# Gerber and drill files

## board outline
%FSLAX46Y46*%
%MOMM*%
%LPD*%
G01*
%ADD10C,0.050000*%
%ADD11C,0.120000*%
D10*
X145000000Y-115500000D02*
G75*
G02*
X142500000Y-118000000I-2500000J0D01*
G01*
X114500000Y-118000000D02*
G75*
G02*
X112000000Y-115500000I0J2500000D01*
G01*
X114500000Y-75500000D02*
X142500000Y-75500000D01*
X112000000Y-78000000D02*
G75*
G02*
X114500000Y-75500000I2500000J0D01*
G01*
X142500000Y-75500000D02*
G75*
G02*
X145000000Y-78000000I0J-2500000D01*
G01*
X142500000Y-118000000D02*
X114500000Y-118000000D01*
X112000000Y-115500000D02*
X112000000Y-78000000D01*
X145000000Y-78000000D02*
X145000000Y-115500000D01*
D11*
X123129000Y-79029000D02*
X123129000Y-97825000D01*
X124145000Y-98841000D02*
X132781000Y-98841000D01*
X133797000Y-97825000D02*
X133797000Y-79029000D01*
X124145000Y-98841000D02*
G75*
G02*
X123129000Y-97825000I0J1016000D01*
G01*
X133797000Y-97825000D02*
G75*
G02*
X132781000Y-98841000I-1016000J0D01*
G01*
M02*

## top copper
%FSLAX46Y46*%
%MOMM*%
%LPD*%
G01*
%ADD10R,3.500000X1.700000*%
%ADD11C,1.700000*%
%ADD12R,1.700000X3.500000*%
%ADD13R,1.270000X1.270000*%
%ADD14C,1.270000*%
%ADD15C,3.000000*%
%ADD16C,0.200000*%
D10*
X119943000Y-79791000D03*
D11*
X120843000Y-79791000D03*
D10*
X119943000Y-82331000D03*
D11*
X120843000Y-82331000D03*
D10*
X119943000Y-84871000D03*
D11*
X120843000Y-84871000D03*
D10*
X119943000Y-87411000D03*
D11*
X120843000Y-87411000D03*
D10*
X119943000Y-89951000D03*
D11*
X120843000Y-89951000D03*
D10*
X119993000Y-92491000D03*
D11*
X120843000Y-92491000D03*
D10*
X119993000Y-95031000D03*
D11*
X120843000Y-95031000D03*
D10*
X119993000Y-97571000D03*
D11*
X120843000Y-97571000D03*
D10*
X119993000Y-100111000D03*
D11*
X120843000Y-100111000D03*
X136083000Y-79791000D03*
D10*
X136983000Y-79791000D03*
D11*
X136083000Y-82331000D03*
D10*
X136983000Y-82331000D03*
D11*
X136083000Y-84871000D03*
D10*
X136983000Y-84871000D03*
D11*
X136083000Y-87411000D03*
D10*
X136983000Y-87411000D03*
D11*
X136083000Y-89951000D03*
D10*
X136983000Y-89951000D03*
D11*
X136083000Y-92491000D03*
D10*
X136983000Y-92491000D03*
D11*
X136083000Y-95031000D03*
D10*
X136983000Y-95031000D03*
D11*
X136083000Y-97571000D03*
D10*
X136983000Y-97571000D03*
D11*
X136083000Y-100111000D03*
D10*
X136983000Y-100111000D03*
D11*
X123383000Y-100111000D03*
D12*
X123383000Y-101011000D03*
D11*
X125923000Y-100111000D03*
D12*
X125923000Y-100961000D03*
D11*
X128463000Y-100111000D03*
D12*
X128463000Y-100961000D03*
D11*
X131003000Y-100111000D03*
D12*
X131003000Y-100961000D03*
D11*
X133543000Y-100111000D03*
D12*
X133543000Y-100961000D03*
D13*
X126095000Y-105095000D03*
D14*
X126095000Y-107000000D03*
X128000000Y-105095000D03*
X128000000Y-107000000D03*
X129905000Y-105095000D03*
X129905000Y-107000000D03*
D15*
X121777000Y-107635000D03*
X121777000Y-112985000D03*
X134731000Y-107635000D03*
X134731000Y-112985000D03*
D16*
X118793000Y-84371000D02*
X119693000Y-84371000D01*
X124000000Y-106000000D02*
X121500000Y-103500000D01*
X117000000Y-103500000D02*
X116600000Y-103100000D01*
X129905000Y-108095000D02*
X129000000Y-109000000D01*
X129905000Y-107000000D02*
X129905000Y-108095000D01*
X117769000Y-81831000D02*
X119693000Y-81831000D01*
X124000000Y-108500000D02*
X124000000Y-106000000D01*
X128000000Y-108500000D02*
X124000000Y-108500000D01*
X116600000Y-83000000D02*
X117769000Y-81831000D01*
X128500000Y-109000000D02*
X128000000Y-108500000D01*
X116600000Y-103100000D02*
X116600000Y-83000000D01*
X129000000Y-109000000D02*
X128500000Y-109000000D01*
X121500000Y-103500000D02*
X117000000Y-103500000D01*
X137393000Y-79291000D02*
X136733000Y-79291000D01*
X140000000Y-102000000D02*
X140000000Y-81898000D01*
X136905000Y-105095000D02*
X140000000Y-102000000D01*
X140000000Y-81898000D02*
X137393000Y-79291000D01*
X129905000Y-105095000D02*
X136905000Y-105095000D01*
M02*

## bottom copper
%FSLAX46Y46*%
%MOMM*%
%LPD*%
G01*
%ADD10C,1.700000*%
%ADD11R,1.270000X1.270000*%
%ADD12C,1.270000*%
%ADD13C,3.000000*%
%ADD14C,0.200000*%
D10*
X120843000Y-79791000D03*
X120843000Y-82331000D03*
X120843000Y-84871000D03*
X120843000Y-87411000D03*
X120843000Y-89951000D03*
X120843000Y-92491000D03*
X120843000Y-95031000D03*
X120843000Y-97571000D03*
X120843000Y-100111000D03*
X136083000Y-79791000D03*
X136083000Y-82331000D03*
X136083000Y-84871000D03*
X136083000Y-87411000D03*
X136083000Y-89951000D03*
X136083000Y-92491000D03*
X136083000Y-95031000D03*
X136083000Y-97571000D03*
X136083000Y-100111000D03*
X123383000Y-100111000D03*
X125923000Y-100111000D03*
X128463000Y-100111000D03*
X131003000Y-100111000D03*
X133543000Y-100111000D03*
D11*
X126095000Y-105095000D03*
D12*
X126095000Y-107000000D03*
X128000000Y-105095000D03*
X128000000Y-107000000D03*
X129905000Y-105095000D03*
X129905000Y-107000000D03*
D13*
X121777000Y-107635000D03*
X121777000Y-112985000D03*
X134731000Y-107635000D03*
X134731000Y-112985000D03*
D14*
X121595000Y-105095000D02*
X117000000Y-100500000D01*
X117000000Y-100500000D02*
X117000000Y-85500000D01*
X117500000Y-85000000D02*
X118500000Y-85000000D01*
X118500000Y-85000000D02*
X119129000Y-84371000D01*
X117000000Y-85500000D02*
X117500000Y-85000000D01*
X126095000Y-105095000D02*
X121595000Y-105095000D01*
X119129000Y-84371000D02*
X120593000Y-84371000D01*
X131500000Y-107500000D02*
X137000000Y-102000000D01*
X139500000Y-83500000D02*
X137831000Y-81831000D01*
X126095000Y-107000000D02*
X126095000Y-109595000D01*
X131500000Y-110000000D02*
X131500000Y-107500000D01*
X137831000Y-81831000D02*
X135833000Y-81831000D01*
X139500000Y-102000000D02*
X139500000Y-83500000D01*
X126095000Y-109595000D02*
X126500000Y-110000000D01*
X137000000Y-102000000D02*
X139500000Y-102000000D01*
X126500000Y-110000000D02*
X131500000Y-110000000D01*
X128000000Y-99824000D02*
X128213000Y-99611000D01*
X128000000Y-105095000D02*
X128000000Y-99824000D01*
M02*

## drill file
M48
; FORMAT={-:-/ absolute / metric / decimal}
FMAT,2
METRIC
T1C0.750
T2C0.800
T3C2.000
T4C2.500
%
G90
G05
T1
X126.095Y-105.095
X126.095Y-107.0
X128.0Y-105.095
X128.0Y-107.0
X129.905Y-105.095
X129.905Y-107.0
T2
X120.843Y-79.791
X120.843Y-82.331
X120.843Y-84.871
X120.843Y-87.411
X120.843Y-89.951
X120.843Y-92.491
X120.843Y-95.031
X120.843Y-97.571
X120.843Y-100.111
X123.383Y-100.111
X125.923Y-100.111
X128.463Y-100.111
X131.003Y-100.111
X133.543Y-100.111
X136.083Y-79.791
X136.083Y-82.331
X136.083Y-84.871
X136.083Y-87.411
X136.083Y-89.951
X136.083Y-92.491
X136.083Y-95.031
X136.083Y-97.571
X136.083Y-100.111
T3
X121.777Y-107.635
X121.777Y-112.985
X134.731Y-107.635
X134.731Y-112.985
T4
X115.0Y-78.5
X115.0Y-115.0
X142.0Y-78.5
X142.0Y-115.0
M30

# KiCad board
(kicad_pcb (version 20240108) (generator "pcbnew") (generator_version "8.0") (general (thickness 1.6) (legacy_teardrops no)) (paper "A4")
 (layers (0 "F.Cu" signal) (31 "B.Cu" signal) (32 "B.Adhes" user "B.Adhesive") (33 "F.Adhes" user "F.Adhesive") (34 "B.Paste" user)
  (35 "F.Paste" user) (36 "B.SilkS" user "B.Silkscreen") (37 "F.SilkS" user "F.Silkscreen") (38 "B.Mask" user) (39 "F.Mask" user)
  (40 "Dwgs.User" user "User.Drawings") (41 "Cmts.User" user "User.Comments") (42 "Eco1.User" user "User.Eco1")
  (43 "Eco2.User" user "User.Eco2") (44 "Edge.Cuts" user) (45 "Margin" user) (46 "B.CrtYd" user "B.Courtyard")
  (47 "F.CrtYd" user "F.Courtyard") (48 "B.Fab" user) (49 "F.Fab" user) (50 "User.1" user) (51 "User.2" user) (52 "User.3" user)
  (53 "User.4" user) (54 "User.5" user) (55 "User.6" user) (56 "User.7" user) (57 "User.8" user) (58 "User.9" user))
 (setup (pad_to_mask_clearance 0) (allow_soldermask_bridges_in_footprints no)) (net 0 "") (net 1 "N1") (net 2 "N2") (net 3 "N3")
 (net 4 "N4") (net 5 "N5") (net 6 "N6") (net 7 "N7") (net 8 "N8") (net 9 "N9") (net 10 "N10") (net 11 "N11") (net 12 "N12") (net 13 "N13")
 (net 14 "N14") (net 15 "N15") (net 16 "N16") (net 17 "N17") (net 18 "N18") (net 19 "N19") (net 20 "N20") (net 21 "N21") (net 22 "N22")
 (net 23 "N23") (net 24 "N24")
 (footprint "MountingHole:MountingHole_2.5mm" (layer "F.Cu") (at 142 115)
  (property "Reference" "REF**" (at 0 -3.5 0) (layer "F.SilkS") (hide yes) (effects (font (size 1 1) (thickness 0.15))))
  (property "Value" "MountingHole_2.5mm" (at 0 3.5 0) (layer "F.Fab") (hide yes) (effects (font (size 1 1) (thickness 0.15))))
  (pad "" np_thru_hole circle (at 0 0) (size 2.5 2.5) (drill 2.5) (layers "*.Cu" "*.Mask")))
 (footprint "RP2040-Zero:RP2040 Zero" (layer "F.Cu") (at 118.303 102.778)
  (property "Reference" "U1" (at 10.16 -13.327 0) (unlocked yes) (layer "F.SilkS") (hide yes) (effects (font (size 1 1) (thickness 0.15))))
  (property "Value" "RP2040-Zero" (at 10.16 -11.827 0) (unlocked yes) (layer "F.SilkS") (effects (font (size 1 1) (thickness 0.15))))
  (fp_line (start 4.826 -23.749) (end 4.826 -4.953) (stroke (width 0.12) (type default)) (layer "Edge.Cuts"))
  (fp_line (start 5.842 -3.937) (end 14.478 -3.937) (stroke (width 0.12) (type default)) (layer "Edge.Cuts"))
  (fp_line (start 15.494 -4.953) (end 15.494 -23.749) (stroke (width 0.12) (type default)) (layer "Edge.Cuts"))
  (fp_arc (start 5.842 -3.937) (mid 5.12358 -4.23458) (end 4.826 -4.953) (stroke (width 0.12) (type default)) (layer "Edge.Cuts"))
  (fp_arc (start 15.494 -4.953) (mid 15.19642 -4.23458) (end 14.478 -3.937) (stroke (width 0.12) (type default)) (layer "Edge.Cuts"))
  (pad "1" smd rect (at 1.64 -22.987) (size 3.5 1.7) (layers "F.Cu" "F.Mask") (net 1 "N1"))
  (pad "1" thru_hole circle (at 2.54 -22.987) (size 1.7 1.7) (drill 0.8) (layers "*.Cu" "*.Mask") (remove_unused_layers no) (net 1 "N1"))
  (pad "2" smd rect (at 1.64 -20.447) (size 3.5 1.7) (layers "F.Cu" "F.Mask") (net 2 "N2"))
  (pad "2" thru_hole circle (at 2.54 -20.447) (size 1.7 1.7) (drill 0.8) (layers "*.Cu" "*.Mask") (remove_unused_layers no) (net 2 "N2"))
  (pad "3" smd rect (at 1.64 -17.907) (size 3.5 1.7) (layers "F.Cu" "F.Mask") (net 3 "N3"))
  (pad "3" thru_hole circle (at 2.54 -17.907) (size 1.7 1.7) (drill 0.8) (layers "*.Cu" "*.Mask") (remove_unused_layers no) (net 3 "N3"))
  (pad "4" smd rect (at 1.64 -15.367) (size 3.5 1.7) (layers "F.Cu" "F.Mask") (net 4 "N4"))
  (pad "4" thru_hole circle (at 2.54 -15.367) (size 1.7 1.7) (drill 0.8) (layers "*.Cu" "*.Mask") (remove_unused_layers no) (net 4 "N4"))
  (pad "5" smd rect (at 1.64 -12.827) (size 3.5 1.7) (layers "F.Cu" "F.Mask") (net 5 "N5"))
  (pad "5" thru_hole circle (at 2.54 -12.827) (size 1.7 1.7) (drill 0.8) (layers "*.Cu" "*.Mask") (remove_unused_layers no) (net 5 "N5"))
  (pad "6" smd rect (at 1.69 -10.287) (size 3.5 1.7) (layers "F.Cu" "F.Mask") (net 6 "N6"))
  (pad "6" thru_hole circle (at 2.54 -10.287) (size 1.7 1.7) (drill 0.8) (layers "*.Cu" "*.Mask") (remove_unused_layers no) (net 6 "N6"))
  (pad "7" smd rect (at 1.69 -7.747) (size 3.5 1.7) (layers "F.Cu" "F.Mask") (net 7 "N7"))
  (pad "7" thru_hole circle (at 2.54 -7.747) (size 1.7 1.7) (drill 0.8) (layers "*.Cu" "*.Mask") (remove_unused_layers no) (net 7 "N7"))
  (pad "8" smd rect (at 1.69 -5.207) (size 3.5 1.7) (layers "F.Cu" "F.Mask") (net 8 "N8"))
  (pad "8" thru_hole circle (at 2.54 -5.207) (size 1.7 1.7) (drill 0.8) (layers "*.Cu" "*.Mask") (remove_unused_layers no) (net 8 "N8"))
  (pad "9" smd rect (at 1.69 -2.667) (size 3.5 1.7) (layers "F.Cu" "F.Mask") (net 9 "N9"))
  (pad "9" thru_hole circle (at 2.54 -2.667) (size 1.7 1.7) (drill 0.8) (layers "*.Cu" "*.Mask") (remove_unused_layers no) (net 9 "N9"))
  (pad "10" thru_hole circle (at 17.78 -22.987) (size 1.7 1.7) (drill 0.8) (layers "*.Cu" "*.Mask") (remove_unused_layers no) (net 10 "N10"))
  (pad "10" smd rect (at 18.68 -22.987) (size 3.5 1.7) (layers "F.Cu" "F.Mask") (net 10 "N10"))
  (pad "11" thru_hole circle (at 17.78 -20.447) (size 1.7 1.7) (drill 0.8) (layers "*.Cu" "*.Mask") (remove_unused_layers no) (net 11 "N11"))
  (pad "11" smd rect (at 18.68 -20.447) (size 3.5 1.7) (layers "F.Cu" "F.Mask") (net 11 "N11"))
  (pad "12" thru_hole circle (at 17.78 -17.907) (size 1.7 1.7) (drill 0.8) (layers "*.Cu" "*.Mask") (remove_unused_layers no) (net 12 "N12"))
  (pad "12" smd rect (at 18.68 -17.907) (size 3.5 1.7) (layers "F.Cu" "F.Mask") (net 12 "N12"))
  (pad "13" thru_hole circle (at 17.78 -15.367) (size 1.7 1.7) (drill 0.8) (layers "*.Cu" "*.Mask") (remove_unused_layers no) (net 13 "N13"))
  (pad "13" smd rect (at 18.68 -15.367) (size 3.5 1.7) (layers "F.Cu" "F.Mask") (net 13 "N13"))
  (pad "14" thru_hole circle (at 17.78 -12.827) (size 1.7 1.7) (drill 0.8) (layers "*.Cu" "*.Mask") (remove_unused_layers no) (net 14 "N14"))
  (pad "14" smd rect (at 18.68 -12.827) (size 3.5 1.7) (layers "F.Cu" "F.Mask") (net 14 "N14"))
  (pad "15" thru_hole circle (at 17.78 -10.287) (size 1.7 1.7) (drill 0.8) (layers "*.Cu" "*.Mask") (remove_unused_layers no) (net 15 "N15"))
  (pad "15" smd rect (at 18.68 -10.287) (size 3.5 1.7) (layers "F.Cu" "F.Mask") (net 15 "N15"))
  (pad "16" thru_hole circle (at 17.78 -7.747) (size 1.7 1.7) (drill 0.8) (layers "*.Cu" "*.Mask") (remove_unused_layers no) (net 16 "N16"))
  (pad "16" smd rect (at 18.68 -7.747) (size 3.5 1.7) (layers "F.Cu" "F.Mask") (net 16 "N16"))
  (pad "17" thru_hole circle (at 17.78 -5.207) (size 1.7 1.7) (drill 0.8) (layers "*.Cu" "*.Mask") (remove_unused_layers no) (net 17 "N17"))
  (pad "17" smd rect (at 18.68 -5.207) (size 3.5 1.7) (layers "F.Cu" "F.Mask") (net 17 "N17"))
  (pad "18" thru_hole circle (at 17.78 -2.667) (size 1.7 1.7) (drill 0.8) (layers "*.Cu" "*.Mask") (remove_unused_layers no) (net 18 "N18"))
  (pad "18" smd rect (at 18.68 -2.667) (size 3.5 1.7) (layers "F.Cu" "F.Mask") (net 18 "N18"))
  (pad "19" thru_hole circle (at 5.08 -2.667) (size 1.7 1.7) (drill 0.8) (layers "*.Cu" "*.Mask") (remove_unused_layers no) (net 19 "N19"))
  (pad "19" smd rect (at 5.08 -1.767 90) (size 3.5 1.7) (layers "F.Cu" "F.Mask") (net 19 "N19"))
  (pad "20" thru_hole circle (at 7.62 -2.667) (size 1.7 1.7) (drill 0.8) (layers "*.Cu" "*.Mask") (remove_unused_layers no) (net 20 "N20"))
  (pad "20" smd rect (at 7.62 -1.817 90) (size 3.5 1.7) (layers "F.Cu" "F.Mask") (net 20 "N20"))
  (pad "21" thru_hole circle (at 10.16 -2.667) (size 1.7 1.7) (drill 0.8) (layers "*.Cu" "*.Mask") (remove_unused_layers no) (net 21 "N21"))
  (pad "21" smd rect (at 10.16 -1.817 90) (size 3.5 1.7) (layers "F.Cu" "F.Mask") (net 21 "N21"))
  (pad "22" thru_hole circle (at 12.7 -2.667) (size 1.7 1.7) (drill 0.8) (layers "*.Cu" "*.Mask") (remove_unused_layers no) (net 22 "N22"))
  (pad "22" smd rect (at 12.7 -1.817 90) (size 3.5 1.7) (layers "F.Cu" "F.Mask") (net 22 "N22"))
  (pad "23" thru_hole circle (at 15.24 -2.667) (size 1.7 1.7) (drill 0.8) (layers "*.Cu" "*.Mask") (remove_unused_layers no) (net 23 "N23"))
  (pad "23" smd rect (at 15.24 -1.817 90) (size 3.5 1.7) (layers "F.Cu" "F.Mask") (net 23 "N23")))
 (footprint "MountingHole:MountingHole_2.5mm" (layer "F.Cu") (at 115 115)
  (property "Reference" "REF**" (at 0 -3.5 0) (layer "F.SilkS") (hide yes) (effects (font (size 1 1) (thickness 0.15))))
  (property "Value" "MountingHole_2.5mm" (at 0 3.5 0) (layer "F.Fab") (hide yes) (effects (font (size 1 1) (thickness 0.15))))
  (pad "" np_thru_hole circle (at 0 0) (size 2.5 2.5) (drill 2.5) (layers "*.Cu" "*.Mask")))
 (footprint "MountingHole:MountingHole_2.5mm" (layer "F.Cu") (at 115 78.5)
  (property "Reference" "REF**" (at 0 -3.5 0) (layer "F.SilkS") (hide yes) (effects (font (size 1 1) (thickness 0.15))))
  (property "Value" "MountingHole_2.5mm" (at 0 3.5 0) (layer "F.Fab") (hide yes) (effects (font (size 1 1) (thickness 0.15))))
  (pad "" np_thru_hole circle (at 0 0) (size 2.5 2.5) (drill 2.5) (layers "*.Cu" "*.Mask")))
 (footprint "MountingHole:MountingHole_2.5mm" (layer "F.Cu") (at 142 78.5)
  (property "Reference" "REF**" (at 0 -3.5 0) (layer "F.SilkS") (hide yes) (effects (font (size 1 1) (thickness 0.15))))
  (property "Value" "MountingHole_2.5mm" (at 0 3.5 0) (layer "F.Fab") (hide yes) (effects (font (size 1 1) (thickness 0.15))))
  (pad "" np_thru_hole circle (at 0 0) (size 2.5 2.5) (drill 2.5) (layers "*.Cu" "*.Mask")))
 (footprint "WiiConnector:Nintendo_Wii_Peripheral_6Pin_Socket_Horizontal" (layer "F.Cu") (at 126.095 105.095)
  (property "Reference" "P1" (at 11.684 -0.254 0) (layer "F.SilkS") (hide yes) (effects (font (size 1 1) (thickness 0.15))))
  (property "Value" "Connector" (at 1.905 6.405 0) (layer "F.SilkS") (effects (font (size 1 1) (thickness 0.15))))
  (pad "1" thru_hole rect (at 0 0 180) (size 1.27 1.27) (drill 0.75) (layers "*.Cu" "*.Mask") (remove_unused_layers no) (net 3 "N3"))
  (pad "2" thru_hole circle (at 0 1.905 180) (size 1.27 1.27) (drill 0.75) (layers "*.Cu" "*.Mask") (remove_unused_layers no) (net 11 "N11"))
  (pad "3" thru_hole circle (at 1.905 0 180) (size 1.27 1.27) (drill 0.75) (layers "*.Cu" "*.Mask") (remove_unused_layers no) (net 21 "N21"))
  (pad "4" thru_hole circle (at 1.905 1.905 180) (size 1.27 1.27) (drill 0.75) (layers "*.Cu" "*.Mask") (remove_unused_layers no)
   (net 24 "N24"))
  (pad "5" thru_hole circle (at 3.81 0 180) (size 1.27 1.27) (drill 0.75) (layers "*.Cu" "*.Mask") (remove_unused_layers no) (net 10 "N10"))
  (pad "6" thru_hole circle (at 3.81 1.905 180) (size 1.27 1.27) (drill 0.75) (layers "*.Cu" "*.Mask") (remove_unused_layers no)
   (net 2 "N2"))
  (pad "SH" thru_hole circle (at -4.318 2.54 180) (size 3 3) (drill 2) (layers "*.Cu" "*.Mask") (remove_unused_layers no))
  (pad "SH" thru_hole circle (at -4.318 7.89 180) (size 3 3) (drill 2) (layers "*.Cu" "*.Mask") (remove_unused_layers no))
  (pad "SH" thru_hole circle (at 8.636 2.54 180) (size 3 3) (drill 2) (layers "*.Cu" "*.Mask") (remove_unused_layers no))
  (pad "SH" thru_hole circle (at 8.636 7.89 180) (size 3 3) (drill 2) (layers "*.Cu" "*.Mask") (remove_unused_layers no))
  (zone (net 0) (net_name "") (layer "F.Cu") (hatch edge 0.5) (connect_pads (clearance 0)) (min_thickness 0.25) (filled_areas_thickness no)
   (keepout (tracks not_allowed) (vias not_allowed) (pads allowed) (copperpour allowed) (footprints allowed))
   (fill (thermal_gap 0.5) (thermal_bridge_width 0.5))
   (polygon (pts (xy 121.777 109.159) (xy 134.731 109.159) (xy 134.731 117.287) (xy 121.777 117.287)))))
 (gr_arc (start 145 115.5) (mid 144.267767 117.267767) (end 142.5 118) (stroke (width 0.05) (type default)) (layer "Edge.Cuts"))
 (gr_arc (start 114.5 118) (mid 112.732233 117.267767) (end 112 115.5) (stroke (width 0.05) (type default)) (layer "Edge.Cuts"))
 (gr_line (start 114.5 75.5) (end 142.5 75.5) (stroke (width 0.05) (type default)) (layer "Edge.Cuts"))
 (gr_arc (start 112 78) (mid 112.732233 76.232233) (end 114.5 75.5) (stroke (width 0.05) (type default)) (layer "Edge.Cuts"))
 (gr_arc (start 142.5 75.5) (mid 144.267767 76.232233) (end 145 78) (stroke (width 0.05) (type default)) (layer "Edge.Cuts"))
 (gr_line (start 142.5 118) (end 114.5 118) (stroke (width 0.05) (type default)) (layer "Edge.Cuts"))
 (gr_line (start 112 115.5) (end 112 78) (stroke (width 0.05) (type default)) (layer "Edge.Cuts"))
 (gr_line (start 145 78) (end 145 115.5) (stroke (width 0.05) (type default)) (layer "Edge.Cuts"))
 (segment (start 118.793 84.371) (end 119.693 84.371) (width 0.2) (layer "F.Cu") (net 3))
 (segment (start 121.595 105.095) (end 117 100.5) (width 0.2) (layer "B.Cu") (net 3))
 (segment (start 117 100.5) (end 117 85.5) (width 0.2) (layer "B.Cu") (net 3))
 (segment (start 117.5 85) (end 118.5 85) (width 0.2) (layer "B.Cu") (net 3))
 (segment (start 118.5 85) (end 119.129 84.371) (width 0.2) (layer "B.Cu") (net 3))
 (segment (start 117 85.5) (end 117.5 85) (width 0.2) (layer "B.Cu") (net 3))
 (segment (start 126.095 105.095) (end 121.595 105.095) (width 0.2) (layer "B.Cu") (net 3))
 (segment (start 119.129 84.371) (end 120.593 84.371) (width 0.2) (layer "B.Cu") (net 3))
 (segment (start 124 106) (end 121.5 103.5) (width 0.2) (layer "F.Cu") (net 2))
 (segment (start 117 103.5) (end 116.6 103.1) (width 0.2) (layer "F.Cu") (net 2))
 (segment (start 129.905 108.095) (end 129 109) (width 0.2) (layer "F.Cu") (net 2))
 (segment (start 129.905 107) (end 129.905 108.095) (width 0.2) (layer "F.Cu") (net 2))
 (segment (start 117.769 81.831) (end 119.693 81.831) (width 0.2) (layer "F.Cu") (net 2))
 (segment (start 124 108.5) (end 124 106) (width 0.2) (layer "F.Cu") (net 2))
 (segment (start 128 108.5) (end 124 108.5) (width 0.2) (layer "F.Cu") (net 2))
 (segment (start 116.6 83) (end 117.769 81.831) (width 0.2) (layer "F.Cu") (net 2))
 (segment (start 128.5 109) (end 128 108.5) (width 0.2) (layer "F.Cu") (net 2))
 (segment (start 116.6 103.1) (end 116.6 83) (width 0.2) (layer "F.Cu") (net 2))
 (segment (start 129 109) (end 128.5 109) (width 0.2) (layer "F.Cu") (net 2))
 (segment (start 121.5 103.5) (end 117 103.5) (width 0.2) (layer "F.Cu") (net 2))
 (segment (start 131.5 107.5) (end 137 102) (width 0.2) (layer "B.Cu") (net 11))
 (segment (start 139.5 83.5) (end 137.831 81.831) (width 0.2) (layer "B.Cu") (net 11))
 (segment (start 126.095 107) (end 126.095 109.595) (width 0.2) (layer "B.Cu") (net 11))
 (segment (start 131.5 110) (end 131.5 107.5) (width 0.2) (layer "B.Cu") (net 11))
 (segment (start 137.831 81.831) (end 135.833 81.831) (width 0.2) (layer "B.Cu") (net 11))
 (segment (start 139.5 102) (end 139.5 83.5) (width 0.2) (layer "B.Cu") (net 11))
 (segment (start 126.095 109.595) (end 126.5 110) (width 0.2) (layer "B.Cu") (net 11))
 (segment (start 137 102) (end 139.5 102) (width 0.2) (layer "B.Cu") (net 11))
 (segment (start 126.5 110) (end 131.5 110) (width 0.2) (layer "B.Cu") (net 11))
 (segment (start 128 99.824) (end 128.213 99.611) (width 0.2) (layer "B.Cu") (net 21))
 (segment (start 128 105.095) (end 128 99.824) (width 0.2) (layer "B.Cu") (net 21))
 (segment (start 137.393 79.291) (end 136.733 79.291) (width 0.2) (layer "F.Cu") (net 10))
 (segment (start 140 102) (end 140 81.898) (width 0.2) (layer "F.Cu") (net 10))
 (segment (start 136.905 105.095) (end 140 102) (width 0.2) (layer "F.Cu") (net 10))
 (segment (start 140 81.898) (end 137.393 79.291) (width 0.2) (layer "F.Cu") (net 10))
 (segment (start 129.905 105.095) (end 136.905 105.095) (width 0.2) (layer "F.Cu") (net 10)))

